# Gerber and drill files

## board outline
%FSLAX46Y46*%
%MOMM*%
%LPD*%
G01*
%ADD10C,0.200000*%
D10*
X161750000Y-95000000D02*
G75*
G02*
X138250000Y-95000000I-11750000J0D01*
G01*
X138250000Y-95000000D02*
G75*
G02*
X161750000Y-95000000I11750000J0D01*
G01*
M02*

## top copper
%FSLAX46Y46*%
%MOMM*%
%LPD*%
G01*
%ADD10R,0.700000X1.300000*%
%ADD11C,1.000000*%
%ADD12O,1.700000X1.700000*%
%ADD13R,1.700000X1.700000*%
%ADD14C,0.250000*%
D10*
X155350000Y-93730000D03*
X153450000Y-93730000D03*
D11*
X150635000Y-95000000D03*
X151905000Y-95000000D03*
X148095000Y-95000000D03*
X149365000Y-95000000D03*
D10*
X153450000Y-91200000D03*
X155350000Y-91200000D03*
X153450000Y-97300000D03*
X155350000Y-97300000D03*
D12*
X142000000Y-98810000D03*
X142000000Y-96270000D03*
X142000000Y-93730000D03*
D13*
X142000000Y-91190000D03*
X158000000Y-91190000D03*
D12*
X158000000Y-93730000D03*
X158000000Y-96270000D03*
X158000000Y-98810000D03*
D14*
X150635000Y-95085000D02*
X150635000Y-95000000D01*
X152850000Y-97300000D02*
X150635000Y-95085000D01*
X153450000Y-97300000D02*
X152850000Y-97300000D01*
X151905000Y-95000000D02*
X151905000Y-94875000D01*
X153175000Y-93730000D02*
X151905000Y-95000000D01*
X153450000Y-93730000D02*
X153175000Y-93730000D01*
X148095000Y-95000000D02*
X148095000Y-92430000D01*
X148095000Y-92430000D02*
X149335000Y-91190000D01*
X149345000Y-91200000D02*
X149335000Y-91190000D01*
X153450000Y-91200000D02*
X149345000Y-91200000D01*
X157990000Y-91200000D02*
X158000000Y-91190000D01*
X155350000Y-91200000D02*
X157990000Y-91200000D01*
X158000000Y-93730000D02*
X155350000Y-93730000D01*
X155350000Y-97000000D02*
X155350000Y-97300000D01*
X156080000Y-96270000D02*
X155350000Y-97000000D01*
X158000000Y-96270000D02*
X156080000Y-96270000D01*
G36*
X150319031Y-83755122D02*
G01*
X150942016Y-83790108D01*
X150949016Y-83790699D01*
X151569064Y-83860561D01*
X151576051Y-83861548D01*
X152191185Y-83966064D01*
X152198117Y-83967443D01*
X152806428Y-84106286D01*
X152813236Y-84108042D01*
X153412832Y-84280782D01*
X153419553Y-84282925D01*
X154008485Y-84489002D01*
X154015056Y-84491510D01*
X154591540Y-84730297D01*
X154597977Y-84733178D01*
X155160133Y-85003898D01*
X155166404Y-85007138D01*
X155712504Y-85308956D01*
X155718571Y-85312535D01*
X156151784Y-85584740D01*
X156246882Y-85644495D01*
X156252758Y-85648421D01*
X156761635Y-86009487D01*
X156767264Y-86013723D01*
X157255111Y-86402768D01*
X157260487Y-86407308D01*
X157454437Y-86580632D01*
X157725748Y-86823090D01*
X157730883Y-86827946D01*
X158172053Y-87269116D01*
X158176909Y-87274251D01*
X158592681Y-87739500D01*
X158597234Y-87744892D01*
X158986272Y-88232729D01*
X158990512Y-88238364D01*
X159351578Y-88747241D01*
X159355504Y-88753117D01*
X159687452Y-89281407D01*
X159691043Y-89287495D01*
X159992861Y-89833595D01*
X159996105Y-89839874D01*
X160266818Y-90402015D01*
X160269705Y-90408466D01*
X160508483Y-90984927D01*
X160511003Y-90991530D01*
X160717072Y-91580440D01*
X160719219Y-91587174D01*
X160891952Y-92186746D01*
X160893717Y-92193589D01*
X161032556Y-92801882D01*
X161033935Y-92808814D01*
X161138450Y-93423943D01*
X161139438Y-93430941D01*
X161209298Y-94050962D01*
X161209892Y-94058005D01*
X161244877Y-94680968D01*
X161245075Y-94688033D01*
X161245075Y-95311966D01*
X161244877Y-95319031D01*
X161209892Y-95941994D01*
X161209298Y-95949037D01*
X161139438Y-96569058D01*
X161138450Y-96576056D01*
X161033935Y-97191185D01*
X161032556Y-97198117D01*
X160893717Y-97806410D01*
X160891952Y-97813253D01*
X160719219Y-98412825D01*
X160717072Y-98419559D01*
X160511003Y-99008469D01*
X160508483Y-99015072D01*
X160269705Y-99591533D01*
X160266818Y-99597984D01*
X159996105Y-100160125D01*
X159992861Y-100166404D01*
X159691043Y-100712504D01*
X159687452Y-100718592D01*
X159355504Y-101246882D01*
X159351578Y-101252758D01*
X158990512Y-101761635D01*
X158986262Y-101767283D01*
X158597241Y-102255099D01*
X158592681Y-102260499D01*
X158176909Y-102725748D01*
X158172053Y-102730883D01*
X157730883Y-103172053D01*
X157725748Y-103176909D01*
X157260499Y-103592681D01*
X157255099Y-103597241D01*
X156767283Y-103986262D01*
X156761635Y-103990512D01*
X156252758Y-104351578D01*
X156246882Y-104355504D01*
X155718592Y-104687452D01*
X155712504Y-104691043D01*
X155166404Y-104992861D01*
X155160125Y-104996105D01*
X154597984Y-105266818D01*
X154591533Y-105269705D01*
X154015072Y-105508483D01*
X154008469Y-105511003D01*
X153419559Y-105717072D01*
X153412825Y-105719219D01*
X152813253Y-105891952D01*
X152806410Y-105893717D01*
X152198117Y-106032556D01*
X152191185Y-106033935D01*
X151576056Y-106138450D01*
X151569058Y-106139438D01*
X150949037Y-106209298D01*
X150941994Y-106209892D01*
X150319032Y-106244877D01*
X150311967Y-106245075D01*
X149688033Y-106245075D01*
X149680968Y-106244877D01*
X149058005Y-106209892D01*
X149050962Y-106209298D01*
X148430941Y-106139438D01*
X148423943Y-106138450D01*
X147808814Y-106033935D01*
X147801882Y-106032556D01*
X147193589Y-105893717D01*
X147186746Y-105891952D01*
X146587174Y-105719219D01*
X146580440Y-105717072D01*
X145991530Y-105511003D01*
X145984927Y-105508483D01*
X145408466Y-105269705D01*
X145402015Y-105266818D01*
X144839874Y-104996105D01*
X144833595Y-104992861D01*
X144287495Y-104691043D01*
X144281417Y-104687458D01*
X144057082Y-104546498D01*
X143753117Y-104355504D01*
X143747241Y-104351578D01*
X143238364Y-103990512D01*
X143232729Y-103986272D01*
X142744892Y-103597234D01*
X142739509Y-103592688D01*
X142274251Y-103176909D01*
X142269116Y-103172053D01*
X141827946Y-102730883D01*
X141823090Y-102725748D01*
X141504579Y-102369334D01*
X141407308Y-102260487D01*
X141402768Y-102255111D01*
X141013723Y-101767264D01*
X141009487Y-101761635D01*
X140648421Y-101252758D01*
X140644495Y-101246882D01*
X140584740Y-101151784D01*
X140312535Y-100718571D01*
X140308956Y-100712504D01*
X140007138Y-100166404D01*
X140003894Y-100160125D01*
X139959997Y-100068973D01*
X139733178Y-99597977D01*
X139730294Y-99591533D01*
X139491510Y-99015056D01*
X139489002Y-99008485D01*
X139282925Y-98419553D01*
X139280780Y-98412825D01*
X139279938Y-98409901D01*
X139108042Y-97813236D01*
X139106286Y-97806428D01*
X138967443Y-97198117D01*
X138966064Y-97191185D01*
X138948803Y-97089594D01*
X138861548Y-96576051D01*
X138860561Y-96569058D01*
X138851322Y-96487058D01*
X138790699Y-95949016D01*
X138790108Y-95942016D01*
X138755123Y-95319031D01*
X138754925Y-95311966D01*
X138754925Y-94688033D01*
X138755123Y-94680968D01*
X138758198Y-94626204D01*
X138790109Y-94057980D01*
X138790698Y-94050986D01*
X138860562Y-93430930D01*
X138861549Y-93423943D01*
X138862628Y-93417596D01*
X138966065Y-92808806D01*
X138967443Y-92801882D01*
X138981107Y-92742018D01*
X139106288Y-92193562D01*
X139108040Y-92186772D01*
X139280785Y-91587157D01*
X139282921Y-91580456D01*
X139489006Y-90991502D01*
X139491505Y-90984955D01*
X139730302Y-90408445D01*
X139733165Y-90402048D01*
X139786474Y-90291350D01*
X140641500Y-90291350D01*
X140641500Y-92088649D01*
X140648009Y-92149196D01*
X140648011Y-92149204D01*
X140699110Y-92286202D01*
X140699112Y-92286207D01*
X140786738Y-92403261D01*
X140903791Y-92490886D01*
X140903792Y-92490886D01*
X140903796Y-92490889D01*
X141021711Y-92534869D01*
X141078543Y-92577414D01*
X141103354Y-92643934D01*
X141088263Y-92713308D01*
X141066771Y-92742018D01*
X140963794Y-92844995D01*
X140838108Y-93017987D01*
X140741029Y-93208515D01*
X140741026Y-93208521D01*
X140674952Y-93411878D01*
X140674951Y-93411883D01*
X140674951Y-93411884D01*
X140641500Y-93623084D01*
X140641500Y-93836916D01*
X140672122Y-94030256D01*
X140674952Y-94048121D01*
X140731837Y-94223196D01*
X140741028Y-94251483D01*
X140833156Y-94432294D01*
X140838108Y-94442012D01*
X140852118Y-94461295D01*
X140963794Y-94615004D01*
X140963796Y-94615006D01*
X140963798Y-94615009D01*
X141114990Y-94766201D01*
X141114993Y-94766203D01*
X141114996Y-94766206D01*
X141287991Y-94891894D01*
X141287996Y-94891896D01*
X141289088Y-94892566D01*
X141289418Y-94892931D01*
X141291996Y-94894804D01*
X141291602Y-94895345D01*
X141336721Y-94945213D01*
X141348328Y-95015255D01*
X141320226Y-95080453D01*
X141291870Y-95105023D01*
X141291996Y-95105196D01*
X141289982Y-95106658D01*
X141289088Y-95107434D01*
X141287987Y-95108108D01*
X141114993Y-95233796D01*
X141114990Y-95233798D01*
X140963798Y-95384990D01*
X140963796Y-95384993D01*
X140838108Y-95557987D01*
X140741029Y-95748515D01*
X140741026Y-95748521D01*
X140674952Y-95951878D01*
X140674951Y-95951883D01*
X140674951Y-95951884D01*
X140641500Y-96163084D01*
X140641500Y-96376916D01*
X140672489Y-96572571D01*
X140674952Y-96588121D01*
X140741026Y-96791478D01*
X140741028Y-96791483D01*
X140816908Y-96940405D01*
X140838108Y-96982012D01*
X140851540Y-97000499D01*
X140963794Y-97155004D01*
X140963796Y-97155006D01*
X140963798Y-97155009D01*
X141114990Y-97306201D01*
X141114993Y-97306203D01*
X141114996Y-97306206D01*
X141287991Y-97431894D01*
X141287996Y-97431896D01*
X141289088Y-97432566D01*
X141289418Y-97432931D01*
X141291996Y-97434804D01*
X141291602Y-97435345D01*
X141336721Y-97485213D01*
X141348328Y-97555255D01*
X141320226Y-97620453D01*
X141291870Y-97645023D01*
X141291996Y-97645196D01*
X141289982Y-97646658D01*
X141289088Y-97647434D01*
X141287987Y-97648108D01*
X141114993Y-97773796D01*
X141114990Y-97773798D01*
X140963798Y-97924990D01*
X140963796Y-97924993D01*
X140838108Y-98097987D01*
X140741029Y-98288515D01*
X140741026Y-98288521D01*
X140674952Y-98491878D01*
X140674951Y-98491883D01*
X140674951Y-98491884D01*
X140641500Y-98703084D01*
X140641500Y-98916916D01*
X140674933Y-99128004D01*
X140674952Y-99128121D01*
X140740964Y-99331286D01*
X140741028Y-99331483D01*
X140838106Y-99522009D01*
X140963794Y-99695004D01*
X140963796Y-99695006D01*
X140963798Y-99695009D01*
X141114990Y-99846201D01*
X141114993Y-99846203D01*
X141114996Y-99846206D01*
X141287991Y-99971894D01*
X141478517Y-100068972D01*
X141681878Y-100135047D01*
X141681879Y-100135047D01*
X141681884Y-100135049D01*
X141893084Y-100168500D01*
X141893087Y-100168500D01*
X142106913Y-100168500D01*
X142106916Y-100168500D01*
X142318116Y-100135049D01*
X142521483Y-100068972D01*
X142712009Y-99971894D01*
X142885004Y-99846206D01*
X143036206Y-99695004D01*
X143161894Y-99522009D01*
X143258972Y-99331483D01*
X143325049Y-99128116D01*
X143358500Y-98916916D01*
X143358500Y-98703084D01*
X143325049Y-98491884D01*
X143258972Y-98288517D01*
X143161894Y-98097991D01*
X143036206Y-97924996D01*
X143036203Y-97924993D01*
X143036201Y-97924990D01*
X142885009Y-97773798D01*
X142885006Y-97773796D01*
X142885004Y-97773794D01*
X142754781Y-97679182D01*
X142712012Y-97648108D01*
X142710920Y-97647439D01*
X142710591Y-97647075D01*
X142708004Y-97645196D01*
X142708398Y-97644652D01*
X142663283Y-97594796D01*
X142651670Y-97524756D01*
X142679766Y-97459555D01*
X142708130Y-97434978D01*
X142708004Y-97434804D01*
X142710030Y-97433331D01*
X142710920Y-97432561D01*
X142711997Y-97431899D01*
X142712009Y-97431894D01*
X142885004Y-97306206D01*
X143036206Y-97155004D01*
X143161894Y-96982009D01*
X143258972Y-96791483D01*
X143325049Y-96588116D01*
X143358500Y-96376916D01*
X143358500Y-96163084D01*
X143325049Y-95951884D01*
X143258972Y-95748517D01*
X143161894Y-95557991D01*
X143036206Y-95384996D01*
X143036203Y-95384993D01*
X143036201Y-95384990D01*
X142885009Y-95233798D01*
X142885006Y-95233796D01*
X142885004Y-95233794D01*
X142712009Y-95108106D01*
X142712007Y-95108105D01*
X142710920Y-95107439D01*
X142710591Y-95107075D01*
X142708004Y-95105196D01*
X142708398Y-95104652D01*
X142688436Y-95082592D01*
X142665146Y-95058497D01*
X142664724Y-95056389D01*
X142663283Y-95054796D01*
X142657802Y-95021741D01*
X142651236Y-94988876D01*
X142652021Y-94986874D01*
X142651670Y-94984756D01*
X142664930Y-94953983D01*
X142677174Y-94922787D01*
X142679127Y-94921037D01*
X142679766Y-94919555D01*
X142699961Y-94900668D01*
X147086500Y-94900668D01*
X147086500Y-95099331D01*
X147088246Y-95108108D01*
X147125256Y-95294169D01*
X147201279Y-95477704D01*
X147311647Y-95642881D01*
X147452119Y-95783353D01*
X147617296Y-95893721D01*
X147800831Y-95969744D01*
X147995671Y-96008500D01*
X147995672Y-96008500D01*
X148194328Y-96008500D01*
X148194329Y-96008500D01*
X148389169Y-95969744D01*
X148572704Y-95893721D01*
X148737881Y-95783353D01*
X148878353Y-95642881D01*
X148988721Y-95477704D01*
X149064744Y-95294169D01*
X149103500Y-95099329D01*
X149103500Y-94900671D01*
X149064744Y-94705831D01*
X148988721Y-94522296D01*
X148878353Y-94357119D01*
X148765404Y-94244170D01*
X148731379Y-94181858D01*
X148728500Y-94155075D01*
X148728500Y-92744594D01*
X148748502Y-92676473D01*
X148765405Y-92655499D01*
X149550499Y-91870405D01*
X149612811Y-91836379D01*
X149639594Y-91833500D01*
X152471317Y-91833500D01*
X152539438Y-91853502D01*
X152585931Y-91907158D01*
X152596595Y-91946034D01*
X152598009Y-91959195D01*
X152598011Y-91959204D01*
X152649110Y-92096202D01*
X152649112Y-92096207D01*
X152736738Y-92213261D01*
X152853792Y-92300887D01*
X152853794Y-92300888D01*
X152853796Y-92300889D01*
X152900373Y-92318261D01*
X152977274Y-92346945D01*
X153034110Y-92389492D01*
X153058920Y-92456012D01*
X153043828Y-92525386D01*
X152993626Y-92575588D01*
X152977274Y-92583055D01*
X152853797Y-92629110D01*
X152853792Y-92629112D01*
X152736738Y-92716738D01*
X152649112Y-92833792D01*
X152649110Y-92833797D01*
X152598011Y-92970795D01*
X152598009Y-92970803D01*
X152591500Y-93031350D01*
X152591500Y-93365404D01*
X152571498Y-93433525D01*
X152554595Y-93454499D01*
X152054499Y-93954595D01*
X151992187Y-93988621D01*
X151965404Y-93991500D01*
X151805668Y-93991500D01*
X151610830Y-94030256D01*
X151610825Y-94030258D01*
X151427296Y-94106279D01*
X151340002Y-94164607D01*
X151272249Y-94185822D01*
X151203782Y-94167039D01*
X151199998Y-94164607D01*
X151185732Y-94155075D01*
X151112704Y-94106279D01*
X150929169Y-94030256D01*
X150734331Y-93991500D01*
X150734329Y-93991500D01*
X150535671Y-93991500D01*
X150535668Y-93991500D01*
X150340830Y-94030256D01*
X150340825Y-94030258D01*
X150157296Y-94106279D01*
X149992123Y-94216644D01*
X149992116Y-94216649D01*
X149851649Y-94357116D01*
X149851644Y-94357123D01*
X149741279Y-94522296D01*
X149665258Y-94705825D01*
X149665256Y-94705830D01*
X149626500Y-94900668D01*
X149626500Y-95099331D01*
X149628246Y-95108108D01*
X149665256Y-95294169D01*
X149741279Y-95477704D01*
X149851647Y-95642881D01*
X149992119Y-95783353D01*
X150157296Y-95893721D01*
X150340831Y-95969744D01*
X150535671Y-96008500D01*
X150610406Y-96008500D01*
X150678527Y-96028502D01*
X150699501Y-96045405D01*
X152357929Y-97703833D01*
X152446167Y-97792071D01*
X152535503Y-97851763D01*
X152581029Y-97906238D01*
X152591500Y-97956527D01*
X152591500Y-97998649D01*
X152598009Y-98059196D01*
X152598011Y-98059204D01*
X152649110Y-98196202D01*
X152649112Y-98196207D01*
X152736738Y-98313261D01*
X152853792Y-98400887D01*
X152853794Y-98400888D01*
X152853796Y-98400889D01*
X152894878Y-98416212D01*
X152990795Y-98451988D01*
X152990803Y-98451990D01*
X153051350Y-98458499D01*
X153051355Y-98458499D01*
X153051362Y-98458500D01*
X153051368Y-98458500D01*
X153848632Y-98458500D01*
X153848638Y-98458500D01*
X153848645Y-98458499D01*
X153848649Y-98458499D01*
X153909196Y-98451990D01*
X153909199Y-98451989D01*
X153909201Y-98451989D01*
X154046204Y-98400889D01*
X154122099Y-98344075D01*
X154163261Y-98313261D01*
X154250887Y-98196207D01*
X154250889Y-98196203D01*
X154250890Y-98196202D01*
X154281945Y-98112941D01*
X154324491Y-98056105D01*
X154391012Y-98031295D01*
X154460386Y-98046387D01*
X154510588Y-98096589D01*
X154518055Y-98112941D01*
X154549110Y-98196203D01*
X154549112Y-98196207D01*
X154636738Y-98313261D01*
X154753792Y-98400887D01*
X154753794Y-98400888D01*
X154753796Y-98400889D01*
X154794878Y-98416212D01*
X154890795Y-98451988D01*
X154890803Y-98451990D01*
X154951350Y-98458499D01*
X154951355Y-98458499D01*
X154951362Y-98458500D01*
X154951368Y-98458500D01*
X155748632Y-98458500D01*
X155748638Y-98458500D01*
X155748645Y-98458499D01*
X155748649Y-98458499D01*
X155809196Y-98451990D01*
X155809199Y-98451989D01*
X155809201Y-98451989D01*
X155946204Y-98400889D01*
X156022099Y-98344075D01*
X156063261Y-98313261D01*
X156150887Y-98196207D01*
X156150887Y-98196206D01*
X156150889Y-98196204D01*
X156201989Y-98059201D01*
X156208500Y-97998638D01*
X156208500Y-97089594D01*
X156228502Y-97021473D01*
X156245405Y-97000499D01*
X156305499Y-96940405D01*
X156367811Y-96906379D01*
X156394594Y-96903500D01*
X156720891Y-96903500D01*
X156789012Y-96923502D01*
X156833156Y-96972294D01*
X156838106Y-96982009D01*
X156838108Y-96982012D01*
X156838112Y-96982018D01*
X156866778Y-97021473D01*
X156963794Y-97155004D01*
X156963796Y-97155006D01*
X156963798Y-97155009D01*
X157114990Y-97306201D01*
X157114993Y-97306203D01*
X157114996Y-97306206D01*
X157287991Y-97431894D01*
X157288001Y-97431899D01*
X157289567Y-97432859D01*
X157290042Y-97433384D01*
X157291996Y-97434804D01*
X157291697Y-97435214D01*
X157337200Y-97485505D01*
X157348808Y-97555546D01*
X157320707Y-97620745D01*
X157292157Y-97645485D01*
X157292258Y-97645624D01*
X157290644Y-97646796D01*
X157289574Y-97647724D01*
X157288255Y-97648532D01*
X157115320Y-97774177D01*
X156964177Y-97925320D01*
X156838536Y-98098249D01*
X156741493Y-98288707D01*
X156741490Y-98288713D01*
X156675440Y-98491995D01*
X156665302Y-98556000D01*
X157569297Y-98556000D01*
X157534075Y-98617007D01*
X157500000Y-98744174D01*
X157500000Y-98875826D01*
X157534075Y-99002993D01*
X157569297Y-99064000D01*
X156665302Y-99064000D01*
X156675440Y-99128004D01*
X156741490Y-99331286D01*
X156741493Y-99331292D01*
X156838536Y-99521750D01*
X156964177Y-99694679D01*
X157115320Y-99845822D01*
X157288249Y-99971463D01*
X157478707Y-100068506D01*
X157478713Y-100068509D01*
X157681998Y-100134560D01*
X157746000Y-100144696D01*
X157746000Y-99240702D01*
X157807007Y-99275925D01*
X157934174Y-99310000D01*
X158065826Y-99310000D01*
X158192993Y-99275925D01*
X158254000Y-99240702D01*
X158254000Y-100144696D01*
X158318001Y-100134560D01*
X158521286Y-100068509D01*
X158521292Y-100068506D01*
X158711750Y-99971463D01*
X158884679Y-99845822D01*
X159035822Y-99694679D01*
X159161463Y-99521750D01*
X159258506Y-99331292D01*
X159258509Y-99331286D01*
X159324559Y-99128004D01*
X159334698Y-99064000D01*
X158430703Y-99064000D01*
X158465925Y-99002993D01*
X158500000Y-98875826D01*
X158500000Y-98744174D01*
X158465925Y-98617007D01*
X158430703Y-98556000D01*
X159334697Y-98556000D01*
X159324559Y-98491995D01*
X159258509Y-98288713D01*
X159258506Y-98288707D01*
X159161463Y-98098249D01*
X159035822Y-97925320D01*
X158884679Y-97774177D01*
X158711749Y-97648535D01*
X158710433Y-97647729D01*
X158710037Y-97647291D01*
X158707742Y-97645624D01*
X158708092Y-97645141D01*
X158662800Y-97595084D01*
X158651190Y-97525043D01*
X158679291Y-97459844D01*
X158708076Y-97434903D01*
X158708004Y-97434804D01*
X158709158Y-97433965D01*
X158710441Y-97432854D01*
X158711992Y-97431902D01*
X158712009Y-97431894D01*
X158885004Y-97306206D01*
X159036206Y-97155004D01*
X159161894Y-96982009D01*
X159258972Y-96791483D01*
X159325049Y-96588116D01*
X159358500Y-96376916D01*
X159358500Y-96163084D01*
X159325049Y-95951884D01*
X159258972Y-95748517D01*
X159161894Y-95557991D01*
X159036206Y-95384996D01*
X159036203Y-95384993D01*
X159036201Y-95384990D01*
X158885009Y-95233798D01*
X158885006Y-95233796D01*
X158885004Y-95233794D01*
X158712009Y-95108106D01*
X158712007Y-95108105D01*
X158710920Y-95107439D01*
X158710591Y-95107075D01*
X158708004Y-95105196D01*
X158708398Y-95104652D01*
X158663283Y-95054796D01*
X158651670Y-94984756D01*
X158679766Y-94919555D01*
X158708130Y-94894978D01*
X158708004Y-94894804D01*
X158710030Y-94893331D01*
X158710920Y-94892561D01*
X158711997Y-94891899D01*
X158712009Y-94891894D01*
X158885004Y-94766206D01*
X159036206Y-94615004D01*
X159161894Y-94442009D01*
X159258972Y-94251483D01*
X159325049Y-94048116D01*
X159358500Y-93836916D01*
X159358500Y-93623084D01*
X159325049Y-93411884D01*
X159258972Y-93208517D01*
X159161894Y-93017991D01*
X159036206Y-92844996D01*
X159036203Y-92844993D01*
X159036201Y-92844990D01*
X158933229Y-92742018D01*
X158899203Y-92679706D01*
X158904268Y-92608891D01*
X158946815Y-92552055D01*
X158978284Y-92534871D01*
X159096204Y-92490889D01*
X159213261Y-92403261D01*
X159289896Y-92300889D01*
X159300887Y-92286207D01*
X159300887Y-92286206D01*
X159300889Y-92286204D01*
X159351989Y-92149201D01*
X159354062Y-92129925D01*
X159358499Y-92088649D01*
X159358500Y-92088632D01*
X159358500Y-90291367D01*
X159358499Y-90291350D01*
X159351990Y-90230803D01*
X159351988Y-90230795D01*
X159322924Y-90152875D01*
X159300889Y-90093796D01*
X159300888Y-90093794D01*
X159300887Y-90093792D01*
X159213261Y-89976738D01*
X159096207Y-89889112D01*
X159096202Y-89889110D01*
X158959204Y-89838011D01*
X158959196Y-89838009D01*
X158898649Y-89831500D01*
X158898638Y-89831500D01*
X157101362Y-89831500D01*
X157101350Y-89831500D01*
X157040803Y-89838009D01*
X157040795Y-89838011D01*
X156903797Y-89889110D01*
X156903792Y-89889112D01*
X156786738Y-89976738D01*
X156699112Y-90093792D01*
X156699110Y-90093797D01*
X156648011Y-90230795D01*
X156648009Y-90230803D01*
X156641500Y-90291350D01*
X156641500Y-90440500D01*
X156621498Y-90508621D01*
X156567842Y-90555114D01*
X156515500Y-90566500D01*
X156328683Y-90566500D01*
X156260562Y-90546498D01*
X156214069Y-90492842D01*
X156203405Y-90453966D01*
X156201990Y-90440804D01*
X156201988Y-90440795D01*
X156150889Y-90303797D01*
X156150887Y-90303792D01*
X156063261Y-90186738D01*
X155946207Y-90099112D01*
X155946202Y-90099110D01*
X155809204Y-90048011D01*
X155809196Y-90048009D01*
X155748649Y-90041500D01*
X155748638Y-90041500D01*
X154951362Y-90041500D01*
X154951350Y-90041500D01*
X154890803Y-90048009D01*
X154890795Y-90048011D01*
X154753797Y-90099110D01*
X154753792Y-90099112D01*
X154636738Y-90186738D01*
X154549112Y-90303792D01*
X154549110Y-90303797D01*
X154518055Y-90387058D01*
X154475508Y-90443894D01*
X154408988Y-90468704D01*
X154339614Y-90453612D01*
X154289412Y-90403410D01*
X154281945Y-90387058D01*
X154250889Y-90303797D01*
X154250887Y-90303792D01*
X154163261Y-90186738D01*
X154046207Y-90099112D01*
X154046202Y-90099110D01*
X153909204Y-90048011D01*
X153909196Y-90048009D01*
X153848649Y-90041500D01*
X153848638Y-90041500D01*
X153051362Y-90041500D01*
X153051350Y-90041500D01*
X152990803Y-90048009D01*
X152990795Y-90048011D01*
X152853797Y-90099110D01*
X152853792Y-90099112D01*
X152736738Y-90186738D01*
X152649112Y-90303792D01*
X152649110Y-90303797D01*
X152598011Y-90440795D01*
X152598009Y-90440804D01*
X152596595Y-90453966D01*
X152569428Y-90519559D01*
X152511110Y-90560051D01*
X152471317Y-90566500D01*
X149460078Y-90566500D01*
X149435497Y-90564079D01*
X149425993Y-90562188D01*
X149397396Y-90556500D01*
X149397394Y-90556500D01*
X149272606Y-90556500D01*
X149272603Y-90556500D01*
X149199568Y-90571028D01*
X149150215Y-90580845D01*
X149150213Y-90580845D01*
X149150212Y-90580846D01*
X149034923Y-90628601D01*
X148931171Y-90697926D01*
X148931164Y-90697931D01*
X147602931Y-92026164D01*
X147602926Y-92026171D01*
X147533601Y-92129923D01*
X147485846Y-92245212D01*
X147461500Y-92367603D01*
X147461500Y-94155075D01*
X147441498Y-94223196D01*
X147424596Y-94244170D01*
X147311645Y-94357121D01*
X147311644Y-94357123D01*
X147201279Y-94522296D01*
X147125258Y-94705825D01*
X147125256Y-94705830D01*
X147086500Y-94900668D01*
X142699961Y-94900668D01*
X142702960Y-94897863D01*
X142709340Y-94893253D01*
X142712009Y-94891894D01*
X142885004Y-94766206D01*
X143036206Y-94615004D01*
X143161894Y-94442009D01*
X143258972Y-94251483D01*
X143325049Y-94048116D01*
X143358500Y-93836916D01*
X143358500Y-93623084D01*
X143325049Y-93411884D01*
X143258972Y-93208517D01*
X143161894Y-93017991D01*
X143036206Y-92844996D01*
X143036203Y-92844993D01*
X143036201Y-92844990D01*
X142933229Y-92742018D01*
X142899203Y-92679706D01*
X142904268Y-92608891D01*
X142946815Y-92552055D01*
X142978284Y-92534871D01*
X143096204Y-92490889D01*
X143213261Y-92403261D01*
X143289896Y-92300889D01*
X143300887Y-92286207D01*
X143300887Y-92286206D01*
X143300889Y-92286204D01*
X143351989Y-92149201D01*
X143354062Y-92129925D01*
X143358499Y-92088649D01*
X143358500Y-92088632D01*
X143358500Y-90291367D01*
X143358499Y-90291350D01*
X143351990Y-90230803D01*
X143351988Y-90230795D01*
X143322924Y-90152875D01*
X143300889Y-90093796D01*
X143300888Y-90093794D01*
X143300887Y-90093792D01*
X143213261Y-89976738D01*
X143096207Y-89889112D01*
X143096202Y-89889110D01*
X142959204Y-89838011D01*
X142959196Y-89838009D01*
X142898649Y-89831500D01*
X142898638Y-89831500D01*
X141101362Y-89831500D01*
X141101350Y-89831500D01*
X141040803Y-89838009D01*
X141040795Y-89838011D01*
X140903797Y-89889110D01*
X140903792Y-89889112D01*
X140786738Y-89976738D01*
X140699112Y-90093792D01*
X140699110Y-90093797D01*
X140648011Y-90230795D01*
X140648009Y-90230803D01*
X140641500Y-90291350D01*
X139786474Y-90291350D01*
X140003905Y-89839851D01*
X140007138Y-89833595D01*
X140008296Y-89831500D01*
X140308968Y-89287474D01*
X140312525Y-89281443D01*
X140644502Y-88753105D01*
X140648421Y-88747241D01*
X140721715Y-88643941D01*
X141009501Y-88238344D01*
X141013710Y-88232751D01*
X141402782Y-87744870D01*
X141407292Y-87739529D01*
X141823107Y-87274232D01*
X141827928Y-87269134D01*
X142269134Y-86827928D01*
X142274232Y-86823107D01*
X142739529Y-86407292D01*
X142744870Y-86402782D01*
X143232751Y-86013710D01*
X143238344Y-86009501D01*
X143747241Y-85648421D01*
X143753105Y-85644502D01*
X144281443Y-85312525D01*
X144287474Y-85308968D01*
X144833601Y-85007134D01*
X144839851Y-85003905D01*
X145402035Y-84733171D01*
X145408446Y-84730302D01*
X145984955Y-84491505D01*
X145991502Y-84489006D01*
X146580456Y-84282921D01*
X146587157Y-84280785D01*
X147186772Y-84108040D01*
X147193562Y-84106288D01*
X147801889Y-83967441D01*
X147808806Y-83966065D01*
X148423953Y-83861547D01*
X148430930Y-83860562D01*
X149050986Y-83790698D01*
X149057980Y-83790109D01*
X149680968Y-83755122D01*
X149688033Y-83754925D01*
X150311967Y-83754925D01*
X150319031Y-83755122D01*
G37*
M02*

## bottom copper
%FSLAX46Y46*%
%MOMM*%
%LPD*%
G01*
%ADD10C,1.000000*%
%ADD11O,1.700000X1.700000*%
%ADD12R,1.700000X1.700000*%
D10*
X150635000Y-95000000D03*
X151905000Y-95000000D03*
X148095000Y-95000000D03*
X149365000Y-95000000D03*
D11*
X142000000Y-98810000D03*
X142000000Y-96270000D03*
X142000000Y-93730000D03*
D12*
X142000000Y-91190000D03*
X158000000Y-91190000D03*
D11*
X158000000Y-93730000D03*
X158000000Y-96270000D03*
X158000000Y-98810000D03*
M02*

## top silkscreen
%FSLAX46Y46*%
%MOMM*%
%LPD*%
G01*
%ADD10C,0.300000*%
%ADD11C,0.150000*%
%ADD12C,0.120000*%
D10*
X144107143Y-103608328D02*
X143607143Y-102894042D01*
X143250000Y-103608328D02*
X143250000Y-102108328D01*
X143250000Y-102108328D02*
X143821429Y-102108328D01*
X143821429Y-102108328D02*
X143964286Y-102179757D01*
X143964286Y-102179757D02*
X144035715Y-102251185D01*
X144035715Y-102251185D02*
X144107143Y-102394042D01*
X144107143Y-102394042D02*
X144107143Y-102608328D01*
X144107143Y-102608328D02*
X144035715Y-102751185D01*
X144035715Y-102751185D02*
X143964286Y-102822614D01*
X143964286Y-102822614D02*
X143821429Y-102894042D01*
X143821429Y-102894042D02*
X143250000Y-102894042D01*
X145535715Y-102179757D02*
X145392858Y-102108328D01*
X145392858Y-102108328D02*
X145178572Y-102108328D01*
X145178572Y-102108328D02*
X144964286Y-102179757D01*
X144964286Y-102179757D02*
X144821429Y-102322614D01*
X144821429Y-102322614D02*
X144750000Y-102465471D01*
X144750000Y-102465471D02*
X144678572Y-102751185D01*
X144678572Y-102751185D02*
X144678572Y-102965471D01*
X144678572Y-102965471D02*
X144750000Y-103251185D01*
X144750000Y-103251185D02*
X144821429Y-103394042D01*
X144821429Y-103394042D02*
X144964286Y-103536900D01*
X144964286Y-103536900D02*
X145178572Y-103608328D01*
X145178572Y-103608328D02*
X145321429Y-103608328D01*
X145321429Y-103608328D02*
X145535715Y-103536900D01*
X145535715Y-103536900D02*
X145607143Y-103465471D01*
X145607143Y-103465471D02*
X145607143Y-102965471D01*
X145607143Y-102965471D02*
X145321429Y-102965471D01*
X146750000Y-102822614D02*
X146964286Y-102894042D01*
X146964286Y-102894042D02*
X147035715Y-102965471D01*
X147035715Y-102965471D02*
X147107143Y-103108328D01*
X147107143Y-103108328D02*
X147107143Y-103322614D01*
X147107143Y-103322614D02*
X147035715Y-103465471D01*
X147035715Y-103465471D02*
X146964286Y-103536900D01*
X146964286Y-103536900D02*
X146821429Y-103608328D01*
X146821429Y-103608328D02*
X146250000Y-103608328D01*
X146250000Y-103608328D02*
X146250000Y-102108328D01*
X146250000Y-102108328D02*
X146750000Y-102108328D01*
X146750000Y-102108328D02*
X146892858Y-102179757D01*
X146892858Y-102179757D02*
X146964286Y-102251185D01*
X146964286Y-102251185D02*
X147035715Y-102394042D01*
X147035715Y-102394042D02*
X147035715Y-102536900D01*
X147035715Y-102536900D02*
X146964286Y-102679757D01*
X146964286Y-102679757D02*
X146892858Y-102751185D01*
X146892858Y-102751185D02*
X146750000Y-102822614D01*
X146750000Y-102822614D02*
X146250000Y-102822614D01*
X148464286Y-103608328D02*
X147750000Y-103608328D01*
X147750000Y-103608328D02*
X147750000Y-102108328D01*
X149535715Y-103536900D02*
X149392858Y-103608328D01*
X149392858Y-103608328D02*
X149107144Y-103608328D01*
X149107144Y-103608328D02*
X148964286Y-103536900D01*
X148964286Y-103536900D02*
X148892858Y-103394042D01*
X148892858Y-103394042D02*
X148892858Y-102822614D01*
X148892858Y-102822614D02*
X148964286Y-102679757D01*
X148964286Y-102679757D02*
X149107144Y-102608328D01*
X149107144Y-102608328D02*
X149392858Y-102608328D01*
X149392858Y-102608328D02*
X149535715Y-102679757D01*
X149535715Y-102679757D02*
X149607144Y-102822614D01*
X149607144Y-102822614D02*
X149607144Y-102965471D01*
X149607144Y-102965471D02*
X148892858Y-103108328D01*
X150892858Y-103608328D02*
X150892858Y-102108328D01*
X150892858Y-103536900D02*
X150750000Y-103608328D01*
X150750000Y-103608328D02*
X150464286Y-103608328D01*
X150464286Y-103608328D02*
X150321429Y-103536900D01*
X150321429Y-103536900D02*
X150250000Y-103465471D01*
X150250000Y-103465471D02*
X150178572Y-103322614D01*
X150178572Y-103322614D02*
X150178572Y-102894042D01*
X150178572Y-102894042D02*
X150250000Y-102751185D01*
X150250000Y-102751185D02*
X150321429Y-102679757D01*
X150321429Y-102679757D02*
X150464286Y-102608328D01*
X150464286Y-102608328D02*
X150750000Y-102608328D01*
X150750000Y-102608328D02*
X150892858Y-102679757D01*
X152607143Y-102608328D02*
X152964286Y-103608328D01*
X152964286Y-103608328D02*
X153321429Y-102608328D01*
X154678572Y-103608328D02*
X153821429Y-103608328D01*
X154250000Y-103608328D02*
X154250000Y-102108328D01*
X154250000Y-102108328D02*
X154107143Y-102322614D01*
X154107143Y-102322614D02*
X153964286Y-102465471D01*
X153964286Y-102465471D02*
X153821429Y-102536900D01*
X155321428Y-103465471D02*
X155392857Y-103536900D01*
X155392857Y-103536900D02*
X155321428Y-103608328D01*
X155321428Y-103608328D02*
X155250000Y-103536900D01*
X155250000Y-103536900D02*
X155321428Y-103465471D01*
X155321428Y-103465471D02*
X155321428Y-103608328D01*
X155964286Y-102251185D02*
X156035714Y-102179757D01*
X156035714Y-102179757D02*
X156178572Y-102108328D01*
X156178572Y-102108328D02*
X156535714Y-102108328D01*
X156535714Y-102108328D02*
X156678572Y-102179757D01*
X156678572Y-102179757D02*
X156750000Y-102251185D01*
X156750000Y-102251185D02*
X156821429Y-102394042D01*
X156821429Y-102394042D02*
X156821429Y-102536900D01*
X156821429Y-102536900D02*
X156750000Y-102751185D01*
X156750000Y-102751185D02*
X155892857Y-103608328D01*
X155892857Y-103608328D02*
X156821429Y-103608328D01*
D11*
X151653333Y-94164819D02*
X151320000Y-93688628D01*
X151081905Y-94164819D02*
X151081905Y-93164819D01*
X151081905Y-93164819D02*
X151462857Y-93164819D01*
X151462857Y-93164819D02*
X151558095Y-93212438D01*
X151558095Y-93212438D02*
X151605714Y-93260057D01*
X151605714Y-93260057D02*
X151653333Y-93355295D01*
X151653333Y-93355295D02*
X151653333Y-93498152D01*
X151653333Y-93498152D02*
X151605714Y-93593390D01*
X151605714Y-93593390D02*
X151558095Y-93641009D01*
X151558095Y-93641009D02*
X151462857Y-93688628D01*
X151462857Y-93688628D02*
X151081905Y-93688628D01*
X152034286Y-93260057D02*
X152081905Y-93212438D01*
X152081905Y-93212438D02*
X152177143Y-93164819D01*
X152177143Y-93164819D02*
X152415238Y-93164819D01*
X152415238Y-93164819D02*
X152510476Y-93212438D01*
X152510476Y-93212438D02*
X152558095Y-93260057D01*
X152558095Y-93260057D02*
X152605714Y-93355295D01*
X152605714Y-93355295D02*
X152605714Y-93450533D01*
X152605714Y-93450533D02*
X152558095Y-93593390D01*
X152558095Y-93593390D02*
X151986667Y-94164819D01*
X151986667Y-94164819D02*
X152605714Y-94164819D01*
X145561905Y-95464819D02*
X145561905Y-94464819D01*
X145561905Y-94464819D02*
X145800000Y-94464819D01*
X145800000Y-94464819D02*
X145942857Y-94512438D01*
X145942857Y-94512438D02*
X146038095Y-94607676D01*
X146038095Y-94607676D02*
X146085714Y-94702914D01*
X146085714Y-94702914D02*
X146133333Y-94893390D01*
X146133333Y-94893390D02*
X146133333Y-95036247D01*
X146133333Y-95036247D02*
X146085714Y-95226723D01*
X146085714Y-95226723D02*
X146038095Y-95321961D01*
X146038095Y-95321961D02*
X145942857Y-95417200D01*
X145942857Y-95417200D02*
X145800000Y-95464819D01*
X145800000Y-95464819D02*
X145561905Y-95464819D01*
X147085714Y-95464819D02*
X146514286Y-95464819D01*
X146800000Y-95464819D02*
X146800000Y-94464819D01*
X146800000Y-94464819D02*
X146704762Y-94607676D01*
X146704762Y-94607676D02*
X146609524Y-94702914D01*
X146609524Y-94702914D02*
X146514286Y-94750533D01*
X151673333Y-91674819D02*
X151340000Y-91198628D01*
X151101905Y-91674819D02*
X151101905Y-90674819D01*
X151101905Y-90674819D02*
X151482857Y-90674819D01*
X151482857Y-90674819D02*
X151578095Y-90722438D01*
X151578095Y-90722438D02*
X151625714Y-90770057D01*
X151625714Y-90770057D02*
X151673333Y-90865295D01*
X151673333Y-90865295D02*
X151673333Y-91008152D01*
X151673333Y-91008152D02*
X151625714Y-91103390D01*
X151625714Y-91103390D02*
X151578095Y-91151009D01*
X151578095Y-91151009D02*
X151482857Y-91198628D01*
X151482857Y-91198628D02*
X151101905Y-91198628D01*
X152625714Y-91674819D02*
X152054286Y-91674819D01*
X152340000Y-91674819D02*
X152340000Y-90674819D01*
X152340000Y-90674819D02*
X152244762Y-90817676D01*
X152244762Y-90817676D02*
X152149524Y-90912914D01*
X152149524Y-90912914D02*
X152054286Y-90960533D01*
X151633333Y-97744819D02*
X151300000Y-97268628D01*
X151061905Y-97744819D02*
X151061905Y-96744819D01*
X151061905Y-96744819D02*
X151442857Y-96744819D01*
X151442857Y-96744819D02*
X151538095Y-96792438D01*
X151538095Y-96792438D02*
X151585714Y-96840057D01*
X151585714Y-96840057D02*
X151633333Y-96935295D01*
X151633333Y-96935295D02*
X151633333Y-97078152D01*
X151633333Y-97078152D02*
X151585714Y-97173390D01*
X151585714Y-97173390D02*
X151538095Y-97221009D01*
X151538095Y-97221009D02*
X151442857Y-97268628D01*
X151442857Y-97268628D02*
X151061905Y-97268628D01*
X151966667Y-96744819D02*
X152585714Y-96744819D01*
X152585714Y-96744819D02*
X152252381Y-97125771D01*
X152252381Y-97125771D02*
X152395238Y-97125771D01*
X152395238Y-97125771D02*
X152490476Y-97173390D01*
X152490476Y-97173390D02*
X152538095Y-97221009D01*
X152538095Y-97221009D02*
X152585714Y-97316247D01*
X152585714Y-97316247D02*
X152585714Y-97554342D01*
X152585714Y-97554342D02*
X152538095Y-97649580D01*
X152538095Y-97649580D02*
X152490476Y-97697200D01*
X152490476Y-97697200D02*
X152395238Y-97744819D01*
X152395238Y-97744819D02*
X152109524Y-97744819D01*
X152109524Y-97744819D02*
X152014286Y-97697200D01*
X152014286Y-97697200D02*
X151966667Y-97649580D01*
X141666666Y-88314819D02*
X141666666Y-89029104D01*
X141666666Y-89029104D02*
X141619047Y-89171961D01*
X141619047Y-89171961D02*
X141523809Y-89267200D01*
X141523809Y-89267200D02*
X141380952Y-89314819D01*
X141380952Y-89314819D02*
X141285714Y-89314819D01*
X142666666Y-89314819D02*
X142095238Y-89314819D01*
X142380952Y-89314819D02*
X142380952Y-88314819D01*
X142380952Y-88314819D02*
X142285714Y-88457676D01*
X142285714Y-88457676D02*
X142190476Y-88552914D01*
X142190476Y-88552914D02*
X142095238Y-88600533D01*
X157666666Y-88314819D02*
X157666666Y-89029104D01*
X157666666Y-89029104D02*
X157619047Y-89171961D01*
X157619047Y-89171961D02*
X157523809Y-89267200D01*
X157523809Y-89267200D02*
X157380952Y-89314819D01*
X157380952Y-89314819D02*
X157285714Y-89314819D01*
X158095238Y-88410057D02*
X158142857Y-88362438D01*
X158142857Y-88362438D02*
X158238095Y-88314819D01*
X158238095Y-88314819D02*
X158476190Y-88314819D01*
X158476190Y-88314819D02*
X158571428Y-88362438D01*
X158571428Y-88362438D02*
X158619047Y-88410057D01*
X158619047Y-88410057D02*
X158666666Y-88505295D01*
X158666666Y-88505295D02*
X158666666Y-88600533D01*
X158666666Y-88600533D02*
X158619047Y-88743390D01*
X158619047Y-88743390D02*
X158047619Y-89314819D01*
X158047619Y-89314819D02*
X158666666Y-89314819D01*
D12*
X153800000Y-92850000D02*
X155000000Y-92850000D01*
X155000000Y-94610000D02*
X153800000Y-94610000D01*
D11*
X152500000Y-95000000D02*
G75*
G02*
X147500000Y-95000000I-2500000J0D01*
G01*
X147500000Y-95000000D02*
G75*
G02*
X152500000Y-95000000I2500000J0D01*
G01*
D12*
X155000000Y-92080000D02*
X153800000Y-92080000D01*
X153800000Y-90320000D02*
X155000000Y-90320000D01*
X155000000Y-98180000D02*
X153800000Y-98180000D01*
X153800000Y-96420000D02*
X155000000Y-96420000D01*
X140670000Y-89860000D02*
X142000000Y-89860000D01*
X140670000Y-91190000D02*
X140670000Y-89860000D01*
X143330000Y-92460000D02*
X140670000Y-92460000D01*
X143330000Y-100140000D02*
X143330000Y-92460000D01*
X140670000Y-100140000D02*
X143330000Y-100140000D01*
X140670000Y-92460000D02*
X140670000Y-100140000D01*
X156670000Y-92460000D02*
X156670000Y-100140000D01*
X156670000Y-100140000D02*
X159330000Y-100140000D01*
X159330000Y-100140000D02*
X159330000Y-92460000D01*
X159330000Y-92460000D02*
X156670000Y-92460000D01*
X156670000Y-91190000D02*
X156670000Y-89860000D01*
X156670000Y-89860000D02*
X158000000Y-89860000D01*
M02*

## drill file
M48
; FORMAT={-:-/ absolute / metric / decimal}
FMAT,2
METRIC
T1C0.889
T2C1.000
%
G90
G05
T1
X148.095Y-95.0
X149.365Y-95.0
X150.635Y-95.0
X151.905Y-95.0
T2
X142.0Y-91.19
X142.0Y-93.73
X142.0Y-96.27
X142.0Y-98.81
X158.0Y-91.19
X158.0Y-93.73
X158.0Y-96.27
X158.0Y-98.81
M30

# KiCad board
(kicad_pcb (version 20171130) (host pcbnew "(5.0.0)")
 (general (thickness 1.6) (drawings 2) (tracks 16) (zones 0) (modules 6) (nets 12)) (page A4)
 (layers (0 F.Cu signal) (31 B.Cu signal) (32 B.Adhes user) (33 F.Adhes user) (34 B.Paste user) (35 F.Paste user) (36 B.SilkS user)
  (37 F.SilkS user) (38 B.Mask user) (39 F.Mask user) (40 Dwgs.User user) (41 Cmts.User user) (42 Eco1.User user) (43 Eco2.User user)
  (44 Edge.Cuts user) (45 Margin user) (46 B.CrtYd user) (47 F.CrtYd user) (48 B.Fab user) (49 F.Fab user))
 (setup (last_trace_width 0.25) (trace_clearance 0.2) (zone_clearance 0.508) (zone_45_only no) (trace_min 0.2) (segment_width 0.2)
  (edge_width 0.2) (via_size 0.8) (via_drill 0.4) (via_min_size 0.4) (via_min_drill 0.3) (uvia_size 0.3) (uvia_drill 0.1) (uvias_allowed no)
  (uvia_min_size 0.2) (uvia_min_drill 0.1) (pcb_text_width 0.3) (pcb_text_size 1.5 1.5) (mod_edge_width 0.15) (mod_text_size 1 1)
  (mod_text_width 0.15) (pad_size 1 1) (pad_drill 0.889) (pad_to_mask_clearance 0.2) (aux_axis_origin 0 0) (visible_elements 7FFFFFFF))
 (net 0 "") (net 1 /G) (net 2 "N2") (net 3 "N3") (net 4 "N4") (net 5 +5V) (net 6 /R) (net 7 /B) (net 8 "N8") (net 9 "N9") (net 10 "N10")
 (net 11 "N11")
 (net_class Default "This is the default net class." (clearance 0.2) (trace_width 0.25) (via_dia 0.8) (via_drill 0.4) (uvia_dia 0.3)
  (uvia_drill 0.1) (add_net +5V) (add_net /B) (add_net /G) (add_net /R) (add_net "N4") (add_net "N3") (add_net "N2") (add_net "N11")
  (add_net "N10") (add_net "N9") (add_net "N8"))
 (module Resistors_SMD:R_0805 (layer F.Cu) (at 154.4 93.73)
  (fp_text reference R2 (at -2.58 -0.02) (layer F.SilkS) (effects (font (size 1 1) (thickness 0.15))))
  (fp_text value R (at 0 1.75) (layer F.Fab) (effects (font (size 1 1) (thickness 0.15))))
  (fp_line (start -0.6 -0.88) (end 0.6 -0.88) (layer F.SilkS) (width 0.12))
  (fp_line (start 0.6 0.88) (end -0.6 0.88) (layer F.SilkS) (width 0.12))
  (pad 2 smd rect (at 0.95 0) (size 0.7 1.3) (layers F.Cu F.Paste F.Mask) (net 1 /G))
  (pad 1 smd rect (at -0.95 0) (size 0.7 1.3) (layers F.Cu F.Paste F.Mask) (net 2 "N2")))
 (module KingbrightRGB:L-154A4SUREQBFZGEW (layer F.Cu) (at 150 95)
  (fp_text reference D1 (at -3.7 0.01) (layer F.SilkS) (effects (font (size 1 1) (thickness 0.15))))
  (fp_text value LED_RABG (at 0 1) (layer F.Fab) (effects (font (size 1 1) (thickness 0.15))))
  (fp_circle (center 0 0) (end 2.5 0) (layer F.SilkS) (width 0.15))
  (pad 3 thru_hole circle (at 0.635 0) (size 1 1) (drill 0.889) (layers *.Cu *.Mask) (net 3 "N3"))
  (pad 4 thru_hole circle (at 1.905 0) (size 1 1) (drill 0.889) (layers *.Cu *.Mask) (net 2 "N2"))
  (pad 1 thru_hole circle (at -1.905 0) (size 1 1) (drill 0.889) (layers *.Cu *.Mask) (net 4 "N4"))
  (pad 2 thru_hole circle (at -0.635 0) (size 1 1) (drill 0.889) (layers *.Cu *.Mask) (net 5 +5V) (zone_connect 2)))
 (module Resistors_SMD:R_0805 (layer F.Cu) (at 154.4 91.2)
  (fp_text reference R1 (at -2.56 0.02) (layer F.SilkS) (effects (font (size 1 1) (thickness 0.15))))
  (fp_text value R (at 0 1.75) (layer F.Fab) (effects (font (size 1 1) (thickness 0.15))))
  (fp_line (start 0.6 0.88) (end -0.6 0.88) (layer F.SilkS) (width 0.12))
  (fp_line (start -0.6 -0.88) (end 0.6 -0.88) (layer F.SilkS) (width 0.12))
  (pad 1 smd rect (at -0.95 0) (size 0.7 1.3) (layers F.Cu F.Paste F.Mask) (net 4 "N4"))
  (pad 2 smd rect (at 0.95 0) (size 0.7 1.3) (layers F.Cu F.Paste F.Mask) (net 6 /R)))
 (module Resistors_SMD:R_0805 (layer F.Cu) (at 154.4 97.3)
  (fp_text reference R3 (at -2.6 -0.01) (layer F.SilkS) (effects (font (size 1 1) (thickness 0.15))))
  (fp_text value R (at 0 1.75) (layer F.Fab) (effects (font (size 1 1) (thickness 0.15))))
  (fp_line (start 0.6 0.88) (end -0.6 0.88) (layer F.SilkS) (width 0.12))
  (fp_line (start -0.6 -0.88) (end 0.6 -0.88) (layer F.SilkS) (width 0.12))
  (pad 1 smd rect (at -0.95 0) (size 0.7 1.3) (layers F.Cu F.Paste F.Mask) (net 3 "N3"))
  (pad 2 smd rect (at 0.95 0) (size 0.7 1.3) (layers F.Cu F.Paste F.Mask) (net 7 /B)))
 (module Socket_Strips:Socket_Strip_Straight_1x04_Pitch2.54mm (layer F.Cu) (at 142 91.19)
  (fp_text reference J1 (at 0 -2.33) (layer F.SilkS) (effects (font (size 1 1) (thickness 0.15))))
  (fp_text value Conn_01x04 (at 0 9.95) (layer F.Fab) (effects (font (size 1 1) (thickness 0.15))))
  (fp_line (start -1.33 -1.33) (end 0 -1.33) (layer F.SilkS) (width 0.12))
  (fp_line (start -1.33 0) (end -1.33 -1.33) (layer F.SilkS) (width 0.12))
  (fp_line (start 1.33 1.27) (end -1.33 1.27) (layer F.SilkS) (width 0.12))
  (fp_line (start 1.33 8.95) (end 1.33 1.27) (layer F.SilkS) (width 0.12))
  (fp_line (start -1.33 8.95) (end 1.33 8.95) (layer F.SilkS) (width 0.12))
  (fp_line (start -1.33 1.27) (end -1.33 8.95) (layer F.SilkS) (width 0.12))
  (pad 4 thru_hole oval (at 0 7.62) (size 1.7 1.7) (drill 1) (layers *.Cu *.Mask) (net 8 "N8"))
  (pad 3 thru_hole oval (at 0 5.08) (size 1.7 1.7) (drill 1) (layers *.Cu *.Mask) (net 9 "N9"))
  (pad 2 thru_hole oval (at 0 2.54) (size 1.7 1.7) (drill 1) (layers *.Cu *.Mask) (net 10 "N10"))
  (pad 1 thru_hole rect (at 0 0) (size 1.7 1.7) (drill 1) (layers *.Cu *.Mask) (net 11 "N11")))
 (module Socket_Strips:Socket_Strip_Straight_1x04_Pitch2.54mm (layer F.Cu) (at 158 91.19)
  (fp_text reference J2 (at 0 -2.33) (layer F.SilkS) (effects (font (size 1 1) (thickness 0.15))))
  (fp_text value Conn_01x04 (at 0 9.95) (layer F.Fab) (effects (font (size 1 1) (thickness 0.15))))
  (fp_line (start -1.33 1.27) (end -1.33 8.95) (layer F.SilkS) (width 0.12))
  (fp_line (start -1.33 8.95) (end 1.33 8.95) (layer F.SilkS) (width 0.12))
  (fp_line (start 1.33 8.95) (end 1.33 1.27) (layer F.SilkS) (width 0.12))
  (fp_line (start 1.33 1.27) (end -1.33 1.27) (layer F.SilkS) (width 0.12))
  (fp_line (start -1.33 0) (end -1.33 -1.33) (layer F.SilkS) (width 0.12))
  (fp_line (start -1.33 -1.33) (end 0 -1.33) (layer F.SilkS) (width 0.12))
  (pad 1 thru_hole rect (at 0 0) (size 1.7 1.7) (drill 1) (layers *.Cu *.Mask) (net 6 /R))
  (pad 2 thru_hole oval (at 0 2.54) (size 1.7 1.7) (drill 1) (layers *.Cu *.Mask) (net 1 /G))
  (pad 3 thru_hole oval (at 0 5.08) (size 1.7 1.7) (drill 1) (layers *.Cu *.Mask) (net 7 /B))
  (pad 4 thru_hole oval (at 0 7.62) (size 1.7 1.7) (drill 1) (layers *.Cu *.Mask) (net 5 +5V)))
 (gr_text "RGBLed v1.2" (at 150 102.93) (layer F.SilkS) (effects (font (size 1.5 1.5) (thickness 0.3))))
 (gr_circle (center 150 95) (end 161.75 95) (layer Edge.Cuts) (width 0.2))
 (segment (start 150.635 95.085) (end 150.635 95) (width 0.25) (layer F.Cu) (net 3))
 (segment (start 152.85 97.3) (end 150.635 95.085) (width 0.25) (layer F.Cu) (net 3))
 (segment (start 153.45 97.3) (end 152.85 97.3) (width 0.25) (layer F.Cu) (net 3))
 (segment (start 151.905 95) (end 151.905 94.875) (width 0.25) (layer F.Cu) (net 2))
 (segment (start 153.175 93.73) (end 151.905 95) (width 0.25) (layer F.Cu) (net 2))
 (segment (start 153.45 93.73) (end 153.175 93.73) (width 0.25) (layer F.Cu) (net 2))
 (segment (start 148.095 95) (end 148.095 92.43) (width 0.25) (layer F.Cu) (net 4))
 (segment (start 148.095 92.43) (end 149.335 91.19) (width 0.25) (layer F.Cu) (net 4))
 (segment (start 149.345 91.2) (end 149.335 91.19) (width 0.25) (layer F.Cu) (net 4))
 (segment (start 153.45 91.2) (end 149.345 91.2) (width 0.25) (layer F.Cu) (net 4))
 (segment (start 157.99 91.2) (end 158 91.19) (width 0.25) (layer F.Cu) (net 6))
 (segment (start 155.35 91.2) (end 157.99 91.2) (width 0.25) (layer F.Cu) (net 6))
 (segment (start 158 93.73) (end 155.35 93.73) (width 0.25) (layer F.Cu) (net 1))
 (segment (start 155.35 97) (end 155.35 97.3) (width 0.25) (layer F.Cu) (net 7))
 (segment (start 156.08 96.27) (end 155.35 97) (width 0.25) (layer F.Cu) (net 7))
 (segment (start 158 96.27) (end 156.08 96.27) (width 0.25) (layer F.Cu) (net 7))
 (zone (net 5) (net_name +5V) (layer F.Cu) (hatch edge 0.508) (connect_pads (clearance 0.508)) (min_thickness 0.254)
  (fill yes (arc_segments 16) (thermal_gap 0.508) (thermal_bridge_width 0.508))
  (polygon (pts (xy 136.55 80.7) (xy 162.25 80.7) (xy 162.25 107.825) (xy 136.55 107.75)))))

